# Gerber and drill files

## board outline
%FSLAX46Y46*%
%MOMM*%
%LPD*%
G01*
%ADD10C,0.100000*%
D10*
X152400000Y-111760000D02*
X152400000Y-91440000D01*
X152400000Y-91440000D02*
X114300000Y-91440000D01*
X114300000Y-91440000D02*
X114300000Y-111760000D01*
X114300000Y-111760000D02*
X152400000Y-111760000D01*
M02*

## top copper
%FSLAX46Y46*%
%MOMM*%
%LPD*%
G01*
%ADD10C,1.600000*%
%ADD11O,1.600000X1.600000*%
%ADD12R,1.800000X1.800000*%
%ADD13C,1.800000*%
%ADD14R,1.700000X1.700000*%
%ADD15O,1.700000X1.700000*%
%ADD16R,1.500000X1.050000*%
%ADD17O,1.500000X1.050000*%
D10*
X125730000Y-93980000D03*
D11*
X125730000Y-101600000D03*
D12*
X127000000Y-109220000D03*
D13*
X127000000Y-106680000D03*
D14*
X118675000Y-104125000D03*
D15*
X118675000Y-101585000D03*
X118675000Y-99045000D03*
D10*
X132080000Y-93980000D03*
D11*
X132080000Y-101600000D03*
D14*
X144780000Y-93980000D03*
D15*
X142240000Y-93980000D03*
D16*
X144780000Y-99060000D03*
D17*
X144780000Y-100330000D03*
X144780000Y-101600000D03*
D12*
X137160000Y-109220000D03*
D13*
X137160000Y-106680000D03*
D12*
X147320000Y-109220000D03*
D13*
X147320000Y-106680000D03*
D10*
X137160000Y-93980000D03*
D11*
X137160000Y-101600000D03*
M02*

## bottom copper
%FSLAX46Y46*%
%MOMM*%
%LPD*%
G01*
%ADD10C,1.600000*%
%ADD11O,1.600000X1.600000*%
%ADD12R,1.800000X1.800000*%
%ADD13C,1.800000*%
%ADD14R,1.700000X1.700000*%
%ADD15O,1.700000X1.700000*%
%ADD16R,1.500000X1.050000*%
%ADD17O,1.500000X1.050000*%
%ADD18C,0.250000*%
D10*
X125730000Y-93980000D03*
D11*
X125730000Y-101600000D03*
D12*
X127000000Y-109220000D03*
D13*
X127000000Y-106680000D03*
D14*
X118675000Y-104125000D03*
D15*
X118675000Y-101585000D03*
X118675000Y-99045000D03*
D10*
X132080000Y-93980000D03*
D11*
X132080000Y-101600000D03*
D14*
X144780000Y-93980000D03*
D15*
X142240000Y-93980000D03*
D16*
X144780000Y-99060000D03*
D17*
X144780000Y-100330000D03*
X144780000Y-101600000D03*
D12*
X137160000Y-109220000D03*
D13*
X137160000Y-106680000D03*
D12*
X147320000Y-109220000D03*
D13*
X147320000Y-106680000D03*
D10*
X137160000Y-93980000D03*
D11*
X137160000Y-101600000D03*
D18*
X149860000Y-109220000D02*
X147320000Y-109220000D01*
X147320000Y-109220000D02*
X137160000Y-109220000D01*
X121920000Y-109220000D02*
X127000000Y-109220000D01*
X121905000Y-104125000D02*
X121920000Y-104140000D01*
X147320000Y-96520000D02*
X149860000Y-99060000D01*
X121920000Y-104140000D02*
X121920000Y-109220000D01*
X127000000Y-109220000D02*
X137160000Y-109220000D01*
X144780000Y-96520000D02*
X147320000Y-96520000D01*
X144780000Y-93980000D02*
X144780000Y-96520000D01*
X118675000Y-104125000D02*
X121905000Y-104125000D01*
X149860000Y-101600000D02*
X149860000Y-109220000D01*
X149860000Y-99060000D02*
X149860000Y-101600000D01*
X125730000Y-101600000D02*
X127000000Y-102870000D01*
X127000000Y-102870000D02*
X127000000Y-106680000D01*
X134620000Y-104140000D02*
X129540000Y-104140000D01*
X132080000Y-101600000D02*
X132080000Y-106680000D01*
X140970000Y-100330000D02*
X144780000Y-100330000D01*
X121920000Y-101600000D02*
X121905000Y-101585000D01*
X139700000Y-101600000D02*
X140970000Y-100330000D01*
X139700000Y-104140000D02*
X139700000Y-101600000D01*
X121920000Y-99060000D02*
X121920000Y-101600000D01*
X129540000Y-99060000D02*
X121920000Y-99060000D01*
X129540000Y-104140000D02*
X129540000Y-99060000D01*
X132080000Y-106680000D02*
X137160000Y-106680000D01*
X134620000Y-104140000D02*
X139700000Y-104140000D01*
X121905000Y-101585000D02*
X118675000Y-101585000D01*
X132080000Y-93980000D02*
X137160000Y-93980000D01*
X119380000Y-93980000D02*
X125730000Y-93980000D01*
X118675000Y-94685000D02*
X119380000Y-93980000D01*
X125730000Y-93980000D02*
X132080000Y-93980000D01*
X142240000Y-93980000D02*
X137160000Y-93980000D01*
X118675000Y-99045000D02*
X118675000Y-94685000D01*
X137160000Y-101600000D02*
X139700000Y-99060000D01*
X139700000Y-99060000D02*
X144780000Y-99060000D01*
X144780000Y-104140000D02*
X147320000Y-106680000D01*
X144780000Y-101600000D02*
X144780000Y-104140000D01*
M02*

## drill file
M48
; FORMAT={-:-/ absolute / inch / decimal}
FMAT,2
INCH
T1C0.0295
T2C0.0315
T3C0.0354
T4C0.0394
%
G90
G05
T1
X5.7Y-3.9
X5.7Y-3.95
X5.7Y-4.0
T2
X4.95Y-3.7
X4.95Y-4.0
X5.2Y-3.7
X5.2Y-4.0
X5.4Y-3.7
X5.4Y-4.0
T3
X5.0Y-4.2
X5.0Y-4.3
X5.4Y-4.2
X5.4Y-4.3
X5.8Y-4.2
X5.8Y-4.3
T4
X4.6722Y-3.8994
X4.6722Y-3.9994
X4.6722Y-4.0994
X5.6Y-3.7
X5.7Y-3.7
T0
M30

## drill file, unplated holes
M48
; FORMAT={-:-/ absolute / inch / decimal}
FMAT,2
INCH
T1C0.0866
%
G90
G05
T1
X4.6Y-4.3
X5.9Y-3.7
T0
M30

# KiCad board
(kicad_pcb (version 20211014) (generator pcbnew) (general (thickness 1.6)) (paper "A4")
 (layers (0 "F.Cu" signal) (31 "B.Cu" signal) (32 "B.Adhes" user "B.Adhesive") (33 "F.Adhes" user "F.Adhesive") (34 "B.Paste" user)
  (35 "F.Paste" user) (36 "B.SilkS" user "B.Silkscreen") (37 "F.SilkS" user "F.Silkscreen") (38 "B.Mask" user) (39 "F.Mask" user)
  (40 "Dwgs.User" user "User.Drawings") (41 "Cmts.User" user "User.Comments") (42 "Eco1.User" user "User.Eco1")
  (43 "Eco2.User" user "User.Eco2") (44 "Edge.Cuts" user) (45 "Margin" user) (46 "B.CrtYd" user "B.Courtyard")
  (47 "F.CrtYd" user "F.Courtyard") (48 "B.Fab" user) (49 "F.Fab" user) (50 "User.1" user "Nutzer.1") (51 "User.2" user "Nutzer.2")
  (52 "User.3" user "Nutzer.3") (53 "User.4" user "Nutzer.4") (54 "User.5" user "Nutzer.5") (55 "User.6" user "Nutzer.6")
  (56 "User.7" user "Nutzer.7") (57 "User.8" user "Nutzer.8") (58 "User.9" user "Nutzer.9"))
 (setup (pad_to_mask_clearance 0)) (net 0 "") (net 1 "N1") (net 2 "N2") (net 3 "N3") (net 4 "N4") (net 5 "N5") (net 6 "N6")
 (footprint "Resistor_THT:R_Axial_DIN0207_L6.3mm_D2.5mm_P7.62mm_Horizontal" (layer "F.Cu") (at 125.73 93.98 -90)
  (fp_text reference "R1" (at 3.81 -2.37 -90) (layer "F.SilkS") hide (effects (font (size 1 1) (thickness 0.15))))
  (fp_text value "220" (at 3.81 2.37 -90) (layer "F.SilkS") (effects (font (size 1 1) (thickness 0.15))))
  (pad "1" thru_hole circle (at 0 0 270) (size 1.6 1.6) (drill 0.8) (layers *.Cu *.Mask) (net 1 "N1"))
  (pad "2" thru_hole oval (at 7.62 0 270) (size 1.6 1.6) (drill 0.8) (layers *.Cu *.Mask) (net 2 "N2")))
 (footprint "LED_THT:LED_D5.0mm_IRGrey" (layer "F.Cu") (at 127 109.22 90)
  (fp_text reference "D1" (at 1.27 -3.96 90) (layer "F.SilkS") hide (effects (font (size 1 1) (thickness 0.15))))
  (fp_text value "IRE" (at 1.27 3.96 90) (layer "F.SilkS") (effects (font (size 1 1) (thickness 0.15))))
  (pad "1" thru_hole rect (at 0 0 90) (size 1.8 1.8) (drill 0.9) (layers *.Cu *.Mask) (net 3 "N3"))
  (pad "2" thru_hole circle (at 2.54 0 90) (size 1.8 1.8) (drill 0.9) (layers *.Cu *.Mask) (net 2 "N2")))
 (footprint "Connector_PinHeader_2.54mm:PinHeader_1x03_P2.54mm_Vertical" (layer "F.Cu") (at 118.675 104.125 180)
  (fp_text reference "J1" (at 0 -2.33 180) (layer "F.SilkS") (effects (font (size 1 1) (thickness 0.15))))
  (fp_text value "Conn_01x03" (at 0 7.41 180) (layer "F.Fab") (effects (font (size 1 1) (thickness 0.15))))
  (pad "1" thru_hole rect (at 0 0 180) (size 1.7 1.7) (drill 1) (layers *.Cu *.Mask) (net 3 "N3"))
  (pad "2" thru_hole oval (at 0 2.54 180) (size 1.7 1.7) (drill 1) (layers *.Cu *.Mask) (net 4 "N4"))
  (pad "3" thru_hole oval (at 0 5.08 180) (size 1.7 1.7) (drill 1) (layers *.Cu *.Mask) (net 1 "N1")))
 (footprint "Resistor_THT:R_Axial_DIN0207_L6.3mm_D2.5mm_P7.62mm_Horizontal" (layer "F.Cu") (at 132.08 93.98 -90)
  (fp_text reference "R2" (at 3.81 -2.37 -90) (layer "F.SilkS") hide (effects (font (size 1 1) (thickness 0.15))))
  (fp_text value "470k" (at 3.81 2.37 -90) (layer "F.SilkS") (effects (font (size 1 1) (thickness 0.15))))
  (pad "1" thru_hole circle (at 0 0 270) (size 1.6 1.6) (drill 0.8) (layers *.Cu *.Mask) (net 1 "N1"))
  (pad "2" thru_hole oval (at 7.62 0 270) (size 1.6 1.6) (drill 0.8) (layers *.Cu *.Mask) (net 4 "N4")))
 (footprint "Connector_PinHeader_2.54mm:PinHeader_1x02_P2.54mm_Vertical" (layer "F.Cu") (at 144.78 93.98 -90)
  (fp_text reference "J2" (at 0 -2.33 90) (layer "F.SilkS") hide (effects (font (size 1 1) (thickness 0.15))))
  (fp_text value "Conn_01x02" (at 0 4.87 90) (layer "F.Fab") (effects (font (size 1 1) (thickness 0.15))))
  (pad "1" thru_hole rect (at 0 0 270) (size 1.7 1.7) (drill 1) (layers *.Cu *.Mask) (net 3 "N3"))
  (pad "2" thru_hole oval (at 0 2.54 270) (size 1.7 1.7) (drill 1) (layers *.Cu *.Mask) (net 1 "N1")))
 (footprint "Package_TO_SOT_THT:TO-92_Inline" (layer "F.Cu") (at 144.78 99.06 -90)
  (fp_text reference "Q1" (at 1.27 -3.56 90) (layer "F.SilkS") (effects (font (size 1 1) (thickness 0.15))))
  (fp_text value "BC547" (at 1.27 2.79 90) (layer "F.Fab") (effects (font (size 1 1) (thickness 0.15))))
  (pad "1" thru_hole rect (at 0 0 270) (size 1.05 1.5) (drill 0.75) (layers *.Cu *.Mask) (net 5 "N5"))
  (pad "2" thru_hole oval (at 1.27 0 270) (size 1.05 1.5) (drill 0.75) (layers *.Cu *.Mask) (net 4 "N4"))
  (pad "3" thru_hole oval (at 2.54 0 270) (size 1.05 1.5) (drill 0.75) (layers *.Cu *.Mask) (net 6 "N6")))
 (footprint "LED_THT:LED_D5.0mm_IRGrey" (layer "F.Cu") (at 137.16 109.22 90)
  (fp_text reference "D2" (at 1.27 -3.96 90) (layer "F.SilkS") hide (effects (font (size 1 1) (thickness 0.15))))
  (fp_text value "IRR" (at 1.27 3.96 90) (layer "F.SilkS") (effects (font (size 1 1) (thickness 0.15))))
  (pad "1" thru_hole rect (at 0 0 90) (size 1.8 1.8) (drill 0.9) (layers *.Cu *.Mask) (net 3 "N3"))
  (pad "2" thru_hole circle (at 2.54 0 90) (size 1.8 1.8) (drill 0.9) (layers *.Cu *.Mask) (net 4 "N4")))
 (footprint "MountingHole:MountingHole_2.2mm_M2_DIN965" (layer "F.Cu") (at 149.86 93.98 180)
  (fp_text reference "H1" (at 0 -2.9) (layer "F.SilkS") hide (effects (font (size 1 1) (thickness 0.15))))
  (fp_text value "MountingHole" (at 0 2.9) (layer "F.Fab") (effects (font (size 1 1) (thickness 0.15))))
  (pad "" np_thru_hole circle (at 0 0 180) (size 2.2 2.2) (drill 2.2) (layers *.Cu *.Mask)))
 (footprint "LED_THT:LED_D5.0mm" (layer "F.Cu") (at 147.32 109.22 90)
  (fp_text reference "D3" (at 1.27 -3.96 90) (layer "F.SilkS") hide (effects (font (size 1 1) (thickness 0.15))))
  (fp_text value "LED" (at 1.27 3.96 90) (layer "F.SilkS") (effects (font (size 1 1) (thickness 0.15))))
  (pad "1" thru_hole rect (at 0 0 90) (size 1.8 1.8) (drill 0.9) (layers *.Cu *.Mask) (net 3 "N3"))
  (pad "2" thru_hole circle (at 2.54 0 90) (size 1.8 1.8) (drill 0.9) (layers *.Cu *.Mask) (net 6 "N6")))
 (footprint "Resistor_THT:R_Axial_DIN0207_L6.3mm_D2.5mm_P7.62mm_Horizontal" (layer "F.Cu") (at 137.16 93.98 -90)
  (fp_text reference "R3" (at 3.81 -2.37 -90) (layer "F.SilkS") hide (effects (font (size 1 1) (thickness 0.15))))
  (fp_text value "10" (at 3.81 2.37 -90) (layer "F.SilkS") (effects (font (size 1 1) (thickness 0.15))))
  (pad "1" thru_hole circle (at 0 0 270) (size 1.6 1.6) (drill 0.8) (layers *.Cu *.Mask) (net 1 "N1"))
  (pad "2" thru_hole oval (at 7.62 0 270) (size 1.6 1.6) (drill 0.8) (layers *.Cu *.Mask) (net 5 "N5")))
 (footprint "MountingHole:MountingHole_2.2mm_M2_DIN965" (layer "F.Cu") (at 116.84 109.22)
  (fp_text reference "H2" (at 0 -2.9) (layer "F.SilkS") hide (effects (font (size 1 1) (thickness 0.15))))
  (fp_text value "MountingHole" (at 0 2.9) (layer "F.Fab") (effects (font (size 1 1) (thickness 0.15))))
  (pad "" np_thru_hole circle (at 0 0) (size 2.2 2.2) (drill 2.2) (layers *.Cu *.Mask)))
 (gr_line (start 152.4 111.76) (end 152.4 91.44) (layer "Edge.Cuts") (width 0.1))
 (gr_line (start 152.4 91.44) (end 114.3 91.44) (layer "Edge.Cuts") (width 0.1))
 (gr_line (start 114.3 91.44) (end 114.3 111.76) (layer "Edge.Cuts") (width 0.1))
 (gr_line (start 114.3 111.76) (end 152.4 111.76) (layer "Edge.Cuts") (width 0.1))
 (segment (start 149.86 109.22) (end 147.32 109.22) (width 0.25) (layer "B.Cu") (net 3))
 (segment (start 147.32 109.22) (end 137.16 109.22) (width 0.25) (layer "B.Cu") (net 3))
 (segment (start 121.92 109.22) (end 127 109.22) (width 0.25) (layer "B.Cu") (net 3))
 (segment (start 121.905 104.125) (end 121.92 104.14) (width 0.25) (layer "B.Cu") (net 3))
 (segment (start 147.32 96.52) (end 149.86 99.06) (width 0.25) (layer "B.Cu") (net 3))
 (segment (start 121.92 104.14) (end 121.92 109.22) (width 0.25) (layer "B.Cu") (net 3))
 (segment (start 127 109.22) (end 137.16 109.22) (width 0.25) (layer "B.Cu") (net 3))
 (segment (start 144.78 96.52) (end 147.32 96.52) (width 0.25) (layer "B.Cu") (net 3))
 (segment (start 144.78 93.98) (end 144.78 96.52) (width 0.25) (layer "B.Cu") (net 3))
 (segment (start 118.675 104.125) (end 121.905 104.125) (width 0.25) (layer "B.Cu") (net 3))
 (segment (start 149.86 101.6) (end 149.86 109.22) (width 0.25) (layer "B.Cu") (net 3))
 (segment (start 149.86 99.06) (end 149.86 101.6) (width 0.25) (layer "B.Cu") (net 3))
 (segment (start 125.73 101.6) (end 127 102.87) (width 0.25) (layer "B.Cu") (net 2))
 (segment (start 127 102.87) (end 127 106.68) (width 0.25) (layer "B.Cu") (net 2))
 (segment (start 134.62 104.14) (end 129.54 104.14) (width 0.25) (layer "B.Cu") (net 4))
 (segment (start 132.08 101.6) (end 132.08 106.68) (width 0.25) (layer "B.Cu") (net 4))
 (segment (start 140.97 100.33) (end 144.78 100.33) (width 0.25) (layer "B.Cu") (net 4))
 (segment (start 121.92 101.6) (end 121.905 101.585) (width 0.25) (layer "B.Cu") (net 4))
 (segment (start 139.7 101.6) (end 140.97 100.33) (width 0.25) (layer "B.Cu") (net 4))
 (segment (start 139.7 104.14) (end 139.7 101.6) (width 0.25) (layer "B.Cu") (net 4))
 (segment (start 121.92 99.06) (end 121.92 101.6) (width 0.25) (layer "B.Cu") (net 4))
 (segment (start 129.54 99.06) (end 121.92 99.06) (width 0.25) (layer "B.Cu") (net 4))
 (segment (start 129.54 104.14) (end 129.54 99.06) (width 0.25) (layer "B.Cu") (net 4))
 (segment (start 132.08 106.68) (end 137.16 106.68) (width 0.25) (layer "B.Cu") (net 4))
 (segment (start 134.62 104.14) (end 139.7 104.14) (width 0.25) (layer "B.Cu") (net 4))
 (segment (start 121.905 101.585) (end 118.675 101.585) (width 0.25) (layer "B.Cu") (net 4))
 (segment (start 132.08 93.98) (end 137.16 93.98) (width 0.25) (layer "B.Cu") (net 1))
 (segment (start 119.38 93.98) (end 125.73 93.98) (width 0.25) (layer "B.Cu") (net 1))
 (segment (start 118.675 94.685) (end 119.38 93.98) (width 0.25) (layer "B.Cu") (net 1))
 (segment (start 125.73 93.98) (end 132.08 93.98) (width 0.25) (layer "B.Cu") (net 1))
 (segment (start 142.24 93.98) (end 137.16 93.98) (width 0.25) (layer "B.Cu") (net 1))
 (segment (start 118.675 99.045) (end 118.675 94.685) (width 0.25) (layer "B.Cu") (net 1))
 (segment (start 137.16 101.6) (end 139.7 99.06) (width 0.25) (layer "B.Cu") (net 5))
 (segment (start 139.7 99.06) (end 144.78 99.06) (width 0.25) (layer "B.Cu") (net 5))
 (segment (start 144.78 104.14) (end 147.32 106.68) (width 0.25) (layer "B.Cu") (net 6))
 (segment (start 144.78 101.6) (end 144.78 104.14) (width 0.25) (layer "B.Cu") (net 6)))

